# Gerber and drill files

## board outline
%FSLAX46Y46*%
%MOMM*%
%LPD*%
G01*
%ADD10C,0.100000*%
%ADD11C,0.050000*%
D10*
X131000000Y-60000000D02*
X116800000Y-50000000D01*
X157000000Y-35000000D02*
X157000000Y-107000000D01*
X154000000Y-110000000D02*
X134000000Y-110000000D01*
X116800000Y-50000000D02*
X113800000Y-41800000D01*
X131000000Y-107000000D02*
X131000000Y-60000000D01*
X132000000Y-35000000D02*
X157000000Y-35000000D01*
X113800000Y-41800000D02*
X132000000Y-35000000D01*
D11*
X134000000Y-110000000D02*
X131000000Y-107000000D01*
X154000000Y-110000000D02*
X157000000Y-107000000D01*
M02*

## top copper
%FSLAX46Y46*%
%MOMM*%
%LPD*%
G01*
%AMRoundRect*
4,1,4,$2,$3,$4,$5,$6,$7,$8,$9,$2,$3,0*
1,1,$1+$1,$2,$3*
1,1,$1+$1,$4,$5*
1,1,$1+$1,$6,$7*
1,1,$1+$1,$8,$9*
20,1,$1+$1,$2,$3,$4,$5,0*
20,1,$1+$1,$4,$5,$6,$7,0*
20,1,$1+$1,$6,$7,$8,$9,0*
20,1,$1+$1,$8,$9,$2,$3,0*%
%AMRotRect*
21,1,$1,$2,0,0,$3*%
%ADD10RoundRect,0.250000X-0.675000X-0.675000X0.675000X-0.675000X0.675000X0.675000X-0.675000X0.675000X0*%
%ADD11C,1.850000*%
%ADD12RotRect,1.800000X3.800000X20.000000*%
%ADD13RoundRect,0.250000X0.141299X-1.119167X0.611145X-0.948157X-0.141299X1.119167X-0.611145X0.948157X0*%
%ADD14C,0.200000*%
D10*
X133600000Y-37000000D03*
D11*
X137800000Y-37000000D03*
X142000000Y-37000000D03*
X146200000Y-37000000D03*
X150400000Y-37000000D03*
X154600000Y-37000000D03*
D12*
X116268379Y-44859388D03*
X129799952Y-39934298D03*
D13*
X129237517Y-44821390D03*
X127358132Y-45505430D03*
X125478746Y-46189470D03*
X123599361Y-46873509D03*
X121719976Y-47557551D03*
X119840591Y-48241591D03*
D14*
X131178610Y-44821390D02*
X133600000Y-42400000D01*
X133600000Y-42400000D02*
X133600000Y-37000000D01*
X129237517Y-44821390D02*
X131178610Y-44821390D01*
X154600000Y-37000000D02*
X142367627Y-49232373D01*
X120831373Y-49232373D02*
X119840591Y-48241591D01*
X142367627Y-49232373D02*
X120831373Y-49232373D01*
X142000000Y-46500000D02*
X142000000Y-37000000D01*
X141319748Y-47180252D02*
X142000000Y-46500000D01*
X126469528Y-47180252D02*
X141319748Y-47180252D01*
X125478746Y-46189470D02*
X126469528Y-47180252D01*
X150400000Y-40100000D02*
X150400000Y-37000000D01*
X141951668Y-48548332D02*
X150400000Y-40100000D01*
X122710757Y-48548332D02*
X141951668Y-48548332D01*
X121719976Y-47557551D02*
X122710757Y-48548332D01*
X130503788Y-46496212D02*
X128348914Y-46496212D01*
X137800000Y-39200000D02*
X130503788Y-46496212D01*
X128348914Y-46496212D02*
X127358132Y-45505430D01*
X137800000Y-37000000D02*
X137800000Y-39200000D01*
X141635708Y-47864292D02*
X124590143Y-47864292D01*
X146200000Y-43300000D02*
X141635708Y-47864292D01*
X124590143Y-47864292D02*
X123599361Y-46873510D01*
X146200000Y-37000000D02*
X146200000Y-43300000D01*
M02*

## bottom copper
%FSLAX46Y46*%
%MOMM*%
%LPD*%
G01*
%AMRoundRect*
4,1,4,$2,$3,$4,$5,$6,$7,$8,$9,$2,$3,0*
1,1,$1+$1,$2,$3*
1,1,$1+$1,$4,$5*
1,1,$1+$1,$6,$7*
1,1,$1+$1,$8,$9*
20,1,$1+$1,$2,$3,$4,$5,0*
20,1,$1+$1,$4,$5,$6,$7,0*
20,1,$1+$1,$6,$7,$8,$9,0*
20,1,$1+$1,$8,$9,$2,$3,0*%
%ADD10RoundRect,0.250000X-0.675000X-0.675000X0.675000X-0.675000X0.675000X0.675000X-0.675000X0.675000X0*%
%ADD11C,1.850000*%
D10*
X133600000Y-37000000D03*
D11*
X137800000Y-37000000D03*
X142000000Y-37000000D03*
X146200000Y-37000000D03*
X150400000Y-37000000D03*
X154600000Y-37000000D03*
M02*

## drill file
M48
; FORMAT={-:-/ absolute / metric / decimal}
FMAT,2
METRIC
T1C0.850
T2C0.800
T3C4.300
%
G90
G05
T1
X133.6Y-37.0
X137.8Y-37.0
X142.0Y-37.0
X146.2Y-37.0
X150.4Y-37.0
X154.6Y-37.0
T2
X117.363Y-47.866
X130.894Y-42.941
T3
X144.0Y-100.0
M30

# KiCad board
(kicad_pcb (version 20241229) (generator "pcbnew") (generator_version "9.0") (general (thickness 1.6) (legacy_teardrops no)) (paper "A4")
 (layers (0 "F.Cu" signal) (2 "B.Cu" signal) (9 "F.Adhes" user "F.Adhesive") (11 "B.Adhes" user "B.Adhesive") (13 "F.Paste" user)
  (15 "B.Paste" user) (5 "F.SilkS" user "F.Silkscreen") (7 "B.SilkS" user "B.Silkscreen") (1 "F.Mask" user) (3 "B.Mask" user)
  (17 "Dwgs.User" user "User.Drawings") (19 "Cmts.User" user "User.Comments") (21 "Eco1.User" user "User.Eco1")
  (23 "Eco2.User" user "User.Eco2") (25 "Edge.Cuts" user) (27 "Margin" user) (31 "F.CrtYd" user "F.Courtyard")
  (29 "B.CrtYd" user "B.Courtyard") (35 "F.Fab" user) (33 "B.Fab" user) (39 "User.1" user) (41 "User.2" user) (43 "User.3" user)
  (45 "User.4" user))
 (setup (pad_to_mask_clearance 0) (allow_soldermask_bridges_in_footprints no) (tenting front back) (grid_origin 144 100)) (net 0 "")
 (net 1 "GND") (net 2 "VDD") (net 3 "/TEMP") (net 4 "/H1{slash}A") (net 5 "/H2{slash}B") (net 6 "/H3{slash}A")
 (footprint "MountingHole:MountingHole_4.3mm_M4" (layer "F.Cu") (at 144 100)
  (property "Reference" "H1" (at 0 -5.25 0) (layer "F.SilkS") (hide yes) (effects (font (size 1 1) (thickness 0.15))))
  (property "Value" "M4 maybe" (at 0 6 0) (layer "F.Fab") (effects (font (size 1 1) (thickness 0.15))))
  (pad "" np_thru_hole circle (at 0 0) (size 4.3 4.3) (drill 4.3) (layers "*.Cu" "*.Mask")))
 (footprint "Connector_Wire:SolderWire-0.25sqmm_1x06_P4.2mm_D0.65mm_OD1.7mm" (layer "F.Cu") (at 133.6 37)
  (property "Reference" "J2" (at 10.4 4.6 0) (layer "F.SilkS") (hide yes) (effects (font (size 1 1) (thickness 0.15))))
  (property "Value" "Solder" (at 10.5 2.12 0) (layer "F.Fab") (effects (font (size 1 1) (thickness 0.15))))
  (pad "1" thru_hole roundrect (at 0 0) (size 1.85 1.85) (drill 0.85) (layers "*.Cu" "*.Mask") (remove_unused_layers no)
   (roundrect_rratio 0.135135) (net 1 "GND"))
  (pad "2" thru_hole circle (at 4.2 0) (size 1.85 1.85) (drill 0.85) (layers "*.Cu" "*.Mask") (remove_unused_layers no) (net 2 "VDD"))
  (pad "3" thru_hole circle (at 8.4 0) (size 1.85 1.85) (drill 0.85) (layers "*.Cu" "*.Mask") (remove_unused_layers no) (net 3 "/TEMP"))
  (pad "4" thru_hole circle (at 12.6 0) (size 1.85 1.85) (drill 0.85) (layers "*.Cu" "*.Mask") (remove_unused_layers no)
   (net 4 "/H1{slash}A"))
  (pad "5" thru_hole circle (at 16.8 0) (size 1.85 1.85) (drill 0.85) (layers "*.Cu" "*.Mask") (remove_unused_layers no)
   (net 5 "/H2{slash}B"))
  (pad "6" thru_hole circle (at 21 0) (size 1.85 1.85) (drill 0.85) (layers "*.Cu" "*.Mask") (remove_unused_layers no) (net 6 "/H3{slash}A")))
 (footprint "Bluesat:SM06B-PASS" (layer "F.Cu") (at 121.768691 38.91998 20)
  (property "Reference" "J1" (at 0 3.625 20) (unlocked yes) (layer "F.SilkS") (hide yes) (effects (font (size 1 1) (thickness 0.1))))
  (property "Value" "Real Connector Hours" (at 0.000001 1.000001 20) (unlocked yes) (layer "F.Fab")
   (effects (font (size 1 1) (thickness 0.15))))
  (pad "" smd rect (at -7.2 3.7 20) (size 1.8 3.8) (layers "F.Cu" "F.Mask" "F.Paste") (thermal_bridge_angle 45))
  (pad "" np_thru_hole circle (at -7.2 6.9 20) (size 0.8 0.8) (drill 0.8) (layers "*.Mask"))
  (pad "" smd rect (at 7.2 3.7 20) (size 1.8 3.8) (layers "F.Cu" "F.Mask" "F.Paste") (thermal_bridge_angle 45))
  (pad "" np_thru_hole circle (at 7.2 6.9 20) (size 0.8 0.8) (drill 0.8) (layers "*.Mask"))
  (pad "1" smd roundrect (at 5 8.1 20) (size 1 2.7) (layers "F.Cu" "F.Mask" "F.Paste") (roundrect_rratio 0.25) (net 1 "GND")
   (thermal_bridge_angle 45))
  (pad "2" smd roundrect (at 3 8.1 20) (size 1 2.7) (layers "F.Cu" "F.Mask" "F.Paste") (roundrect_rratio 0.25) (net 2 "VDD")
   (thermal_bridge_angle 45))
  (pad "3" smd roundrect (at 0.999999 8.1 20) (size 1 2.7) (layers "F.Cu" "F.Mask" "F.Paste") (roundrect_rratio 0.25) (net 3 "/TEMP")
   (thermal_bridge_angle 45))
  (pad "4" smd roundrect (at -1 8.099999 20) (size 1 2.7) (layers "F.Cu" "F.Mask" "F.Paste") (roundrect_rratio 0.25) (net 4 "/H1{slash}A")
   (thermal_bridge_angle 45))
  (pad "5" smd roundrect (at -3 8.1 20) (size 1 2.7) (layers "F.Cu" "F.Mask" "F.Paste") (roundrect_rratio 0.25) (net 5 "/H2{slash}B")
   (thermal_bridge_angle 45))
  (pad "6" smd roundrect (at -5 8.1 20) (size 1 2.7) (layers "F.Cu" "F.Mask" "F.Paste") (roundrect_rratio 0.25) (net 6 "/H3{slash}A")
   (thermal_bridge_angle 45)))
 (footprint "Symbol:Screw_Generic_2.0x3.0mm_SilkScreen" (layer "F.Cu") (at 153 98)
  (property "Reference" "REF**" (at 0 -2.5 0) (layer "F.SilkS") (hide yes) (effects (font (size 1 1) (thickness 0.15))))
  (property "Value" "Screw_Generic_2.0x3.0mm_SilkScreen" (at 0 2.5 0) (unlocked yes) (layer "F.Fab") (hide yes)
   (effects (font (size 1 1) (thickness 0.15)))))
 (gr_line (start 131 60) (end 116.8 50) (stroke (width 0.1) (type solid)) (layer "Edge.Cuts"))
 (gr_line (start 157 35) (end 157 107) (stroke (width 0.1) (type solid)) (layer "Edge.Cuts"))
 (gr_line (start 154 110) (end 134 110) (stroke (width 0.1) (type solid)) (layer "Edge.Cuts"))
 (gr_line (start 116.8 50) (end 113.8 41.8) (stroke (width 0.1) (type solid)) (layer "Edge.Cuts"))
 (gr_line (start 131 107) (end 131 60) (stroke (width 0.1) (type solid)) (layer "Edge.Cuts"))
 (gr_line (start 132 35) (end 157 35) (stroke (width 0.1) (type solid)) (layer "Edge.Cuts"))
 (gr_line (start 113.8 41.8) (end 132 35) (stroke (width 0.1) (type solid)) (layer "Edge.Cuts"))
 (gr_line (start 134 110) (end 131 107) (stroke (width 0.05) (type default)) (layer "Edge.Cuts"))
 (gr_line (start 154 110) (end 157 107) (stroke (width 0.05) (type default)) (layer "Edge.Cuts"))
 (segment (start 131.17861 44.82139) (end 133.6 42.4) (width 0.2) (layer "F.Cu") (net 1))
 (segment (start 133.6 42.4) (end 133.6 37) (width 0.2) (layer "F.Cu") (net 1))
 (segment (start 129.237517 44.82139) (end 131.17861 44.82139) (width 0.2) (layer "F.Cu") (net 1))
 (segment (start 154.6 37) (end 142.367627 49.232373) (width 0.2) (layer "F.Cu") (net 6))
 (segment (start 120.831373 49.232373) (end 119.840591 48.241591) (width 0.2) (layer "F.Cu") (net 6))
 (segment (start 142.367627 49.232373) (end 120.831373 49.232373) (width 0.2) (layer "F.Cu") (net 6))
 (segment (start 142 46.5) (end 142 37) (width 0.2) (layer "F.Cu") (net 3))
 (segment (start 141.319748 47.180252) (end 142 46.5) (width 0.2) (layer "F.Cu") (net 3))
 (segment (start 126.469528 47.180252) (end 141.319748 47.180252) (width 0.2) (layer "F.Cu") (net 3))
 (segment (start 125.478746 46.18947) (end 126.469528 47.180252) (width 0.2) (layer "F.Cu") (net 3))
 (segment (start 150.4 40.1) (end 150.4 37) (width 0.2) (layer "F.Cu") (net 5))
 (segment (start 141.951668 48.548332) (end 150.4 40.1) (width 0.2) (layer "F.Cu") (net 5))
 (segment (start 122.710757 48.548332) (end 141.951668 48.548332) (width 0.2) (layer "F.Cu") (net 5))
 (segment (start 121.719976 47.557551) (end 122.710757 48.548332) (width 0.2) (layer "F.Cu") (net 5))
 (segment (start 130.503788 46.496212) (end 128.348914 46.496212) (width 0.2) (layer "F.Cu") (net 2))
 (segment (start 137.8 39.2) (end 130.503788 46.496212) (width 0.2) (layer "F.Cu") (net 2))
 (segment (start 128.348914 46.496212) (end 127.358132 45.50543) (width 0.2) (layer "F.Cu") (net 2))
 (segment (start 137.8 37) (end 137.8 39.2) (width 0.2) (layer "F.Cu") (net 2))
 (segment (start 141.635708 47.864292) (end 124.590143 47.864292) (width 0.2) (layer "F.Cu") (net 4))
 (segment (start 146.2 43.3) (end 141.635708 47.864292) (width 0.2) (layer "F.Cu") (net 4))
 (segment (start 124.590143 47.864292) (end 123.599361 46.87351) (width 0.2) (layer "F.Cu") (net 4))
 (segment (start 146.2 37) (end 146.2 43.3) (width 0.2) (layer "F.Cu") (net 4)))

